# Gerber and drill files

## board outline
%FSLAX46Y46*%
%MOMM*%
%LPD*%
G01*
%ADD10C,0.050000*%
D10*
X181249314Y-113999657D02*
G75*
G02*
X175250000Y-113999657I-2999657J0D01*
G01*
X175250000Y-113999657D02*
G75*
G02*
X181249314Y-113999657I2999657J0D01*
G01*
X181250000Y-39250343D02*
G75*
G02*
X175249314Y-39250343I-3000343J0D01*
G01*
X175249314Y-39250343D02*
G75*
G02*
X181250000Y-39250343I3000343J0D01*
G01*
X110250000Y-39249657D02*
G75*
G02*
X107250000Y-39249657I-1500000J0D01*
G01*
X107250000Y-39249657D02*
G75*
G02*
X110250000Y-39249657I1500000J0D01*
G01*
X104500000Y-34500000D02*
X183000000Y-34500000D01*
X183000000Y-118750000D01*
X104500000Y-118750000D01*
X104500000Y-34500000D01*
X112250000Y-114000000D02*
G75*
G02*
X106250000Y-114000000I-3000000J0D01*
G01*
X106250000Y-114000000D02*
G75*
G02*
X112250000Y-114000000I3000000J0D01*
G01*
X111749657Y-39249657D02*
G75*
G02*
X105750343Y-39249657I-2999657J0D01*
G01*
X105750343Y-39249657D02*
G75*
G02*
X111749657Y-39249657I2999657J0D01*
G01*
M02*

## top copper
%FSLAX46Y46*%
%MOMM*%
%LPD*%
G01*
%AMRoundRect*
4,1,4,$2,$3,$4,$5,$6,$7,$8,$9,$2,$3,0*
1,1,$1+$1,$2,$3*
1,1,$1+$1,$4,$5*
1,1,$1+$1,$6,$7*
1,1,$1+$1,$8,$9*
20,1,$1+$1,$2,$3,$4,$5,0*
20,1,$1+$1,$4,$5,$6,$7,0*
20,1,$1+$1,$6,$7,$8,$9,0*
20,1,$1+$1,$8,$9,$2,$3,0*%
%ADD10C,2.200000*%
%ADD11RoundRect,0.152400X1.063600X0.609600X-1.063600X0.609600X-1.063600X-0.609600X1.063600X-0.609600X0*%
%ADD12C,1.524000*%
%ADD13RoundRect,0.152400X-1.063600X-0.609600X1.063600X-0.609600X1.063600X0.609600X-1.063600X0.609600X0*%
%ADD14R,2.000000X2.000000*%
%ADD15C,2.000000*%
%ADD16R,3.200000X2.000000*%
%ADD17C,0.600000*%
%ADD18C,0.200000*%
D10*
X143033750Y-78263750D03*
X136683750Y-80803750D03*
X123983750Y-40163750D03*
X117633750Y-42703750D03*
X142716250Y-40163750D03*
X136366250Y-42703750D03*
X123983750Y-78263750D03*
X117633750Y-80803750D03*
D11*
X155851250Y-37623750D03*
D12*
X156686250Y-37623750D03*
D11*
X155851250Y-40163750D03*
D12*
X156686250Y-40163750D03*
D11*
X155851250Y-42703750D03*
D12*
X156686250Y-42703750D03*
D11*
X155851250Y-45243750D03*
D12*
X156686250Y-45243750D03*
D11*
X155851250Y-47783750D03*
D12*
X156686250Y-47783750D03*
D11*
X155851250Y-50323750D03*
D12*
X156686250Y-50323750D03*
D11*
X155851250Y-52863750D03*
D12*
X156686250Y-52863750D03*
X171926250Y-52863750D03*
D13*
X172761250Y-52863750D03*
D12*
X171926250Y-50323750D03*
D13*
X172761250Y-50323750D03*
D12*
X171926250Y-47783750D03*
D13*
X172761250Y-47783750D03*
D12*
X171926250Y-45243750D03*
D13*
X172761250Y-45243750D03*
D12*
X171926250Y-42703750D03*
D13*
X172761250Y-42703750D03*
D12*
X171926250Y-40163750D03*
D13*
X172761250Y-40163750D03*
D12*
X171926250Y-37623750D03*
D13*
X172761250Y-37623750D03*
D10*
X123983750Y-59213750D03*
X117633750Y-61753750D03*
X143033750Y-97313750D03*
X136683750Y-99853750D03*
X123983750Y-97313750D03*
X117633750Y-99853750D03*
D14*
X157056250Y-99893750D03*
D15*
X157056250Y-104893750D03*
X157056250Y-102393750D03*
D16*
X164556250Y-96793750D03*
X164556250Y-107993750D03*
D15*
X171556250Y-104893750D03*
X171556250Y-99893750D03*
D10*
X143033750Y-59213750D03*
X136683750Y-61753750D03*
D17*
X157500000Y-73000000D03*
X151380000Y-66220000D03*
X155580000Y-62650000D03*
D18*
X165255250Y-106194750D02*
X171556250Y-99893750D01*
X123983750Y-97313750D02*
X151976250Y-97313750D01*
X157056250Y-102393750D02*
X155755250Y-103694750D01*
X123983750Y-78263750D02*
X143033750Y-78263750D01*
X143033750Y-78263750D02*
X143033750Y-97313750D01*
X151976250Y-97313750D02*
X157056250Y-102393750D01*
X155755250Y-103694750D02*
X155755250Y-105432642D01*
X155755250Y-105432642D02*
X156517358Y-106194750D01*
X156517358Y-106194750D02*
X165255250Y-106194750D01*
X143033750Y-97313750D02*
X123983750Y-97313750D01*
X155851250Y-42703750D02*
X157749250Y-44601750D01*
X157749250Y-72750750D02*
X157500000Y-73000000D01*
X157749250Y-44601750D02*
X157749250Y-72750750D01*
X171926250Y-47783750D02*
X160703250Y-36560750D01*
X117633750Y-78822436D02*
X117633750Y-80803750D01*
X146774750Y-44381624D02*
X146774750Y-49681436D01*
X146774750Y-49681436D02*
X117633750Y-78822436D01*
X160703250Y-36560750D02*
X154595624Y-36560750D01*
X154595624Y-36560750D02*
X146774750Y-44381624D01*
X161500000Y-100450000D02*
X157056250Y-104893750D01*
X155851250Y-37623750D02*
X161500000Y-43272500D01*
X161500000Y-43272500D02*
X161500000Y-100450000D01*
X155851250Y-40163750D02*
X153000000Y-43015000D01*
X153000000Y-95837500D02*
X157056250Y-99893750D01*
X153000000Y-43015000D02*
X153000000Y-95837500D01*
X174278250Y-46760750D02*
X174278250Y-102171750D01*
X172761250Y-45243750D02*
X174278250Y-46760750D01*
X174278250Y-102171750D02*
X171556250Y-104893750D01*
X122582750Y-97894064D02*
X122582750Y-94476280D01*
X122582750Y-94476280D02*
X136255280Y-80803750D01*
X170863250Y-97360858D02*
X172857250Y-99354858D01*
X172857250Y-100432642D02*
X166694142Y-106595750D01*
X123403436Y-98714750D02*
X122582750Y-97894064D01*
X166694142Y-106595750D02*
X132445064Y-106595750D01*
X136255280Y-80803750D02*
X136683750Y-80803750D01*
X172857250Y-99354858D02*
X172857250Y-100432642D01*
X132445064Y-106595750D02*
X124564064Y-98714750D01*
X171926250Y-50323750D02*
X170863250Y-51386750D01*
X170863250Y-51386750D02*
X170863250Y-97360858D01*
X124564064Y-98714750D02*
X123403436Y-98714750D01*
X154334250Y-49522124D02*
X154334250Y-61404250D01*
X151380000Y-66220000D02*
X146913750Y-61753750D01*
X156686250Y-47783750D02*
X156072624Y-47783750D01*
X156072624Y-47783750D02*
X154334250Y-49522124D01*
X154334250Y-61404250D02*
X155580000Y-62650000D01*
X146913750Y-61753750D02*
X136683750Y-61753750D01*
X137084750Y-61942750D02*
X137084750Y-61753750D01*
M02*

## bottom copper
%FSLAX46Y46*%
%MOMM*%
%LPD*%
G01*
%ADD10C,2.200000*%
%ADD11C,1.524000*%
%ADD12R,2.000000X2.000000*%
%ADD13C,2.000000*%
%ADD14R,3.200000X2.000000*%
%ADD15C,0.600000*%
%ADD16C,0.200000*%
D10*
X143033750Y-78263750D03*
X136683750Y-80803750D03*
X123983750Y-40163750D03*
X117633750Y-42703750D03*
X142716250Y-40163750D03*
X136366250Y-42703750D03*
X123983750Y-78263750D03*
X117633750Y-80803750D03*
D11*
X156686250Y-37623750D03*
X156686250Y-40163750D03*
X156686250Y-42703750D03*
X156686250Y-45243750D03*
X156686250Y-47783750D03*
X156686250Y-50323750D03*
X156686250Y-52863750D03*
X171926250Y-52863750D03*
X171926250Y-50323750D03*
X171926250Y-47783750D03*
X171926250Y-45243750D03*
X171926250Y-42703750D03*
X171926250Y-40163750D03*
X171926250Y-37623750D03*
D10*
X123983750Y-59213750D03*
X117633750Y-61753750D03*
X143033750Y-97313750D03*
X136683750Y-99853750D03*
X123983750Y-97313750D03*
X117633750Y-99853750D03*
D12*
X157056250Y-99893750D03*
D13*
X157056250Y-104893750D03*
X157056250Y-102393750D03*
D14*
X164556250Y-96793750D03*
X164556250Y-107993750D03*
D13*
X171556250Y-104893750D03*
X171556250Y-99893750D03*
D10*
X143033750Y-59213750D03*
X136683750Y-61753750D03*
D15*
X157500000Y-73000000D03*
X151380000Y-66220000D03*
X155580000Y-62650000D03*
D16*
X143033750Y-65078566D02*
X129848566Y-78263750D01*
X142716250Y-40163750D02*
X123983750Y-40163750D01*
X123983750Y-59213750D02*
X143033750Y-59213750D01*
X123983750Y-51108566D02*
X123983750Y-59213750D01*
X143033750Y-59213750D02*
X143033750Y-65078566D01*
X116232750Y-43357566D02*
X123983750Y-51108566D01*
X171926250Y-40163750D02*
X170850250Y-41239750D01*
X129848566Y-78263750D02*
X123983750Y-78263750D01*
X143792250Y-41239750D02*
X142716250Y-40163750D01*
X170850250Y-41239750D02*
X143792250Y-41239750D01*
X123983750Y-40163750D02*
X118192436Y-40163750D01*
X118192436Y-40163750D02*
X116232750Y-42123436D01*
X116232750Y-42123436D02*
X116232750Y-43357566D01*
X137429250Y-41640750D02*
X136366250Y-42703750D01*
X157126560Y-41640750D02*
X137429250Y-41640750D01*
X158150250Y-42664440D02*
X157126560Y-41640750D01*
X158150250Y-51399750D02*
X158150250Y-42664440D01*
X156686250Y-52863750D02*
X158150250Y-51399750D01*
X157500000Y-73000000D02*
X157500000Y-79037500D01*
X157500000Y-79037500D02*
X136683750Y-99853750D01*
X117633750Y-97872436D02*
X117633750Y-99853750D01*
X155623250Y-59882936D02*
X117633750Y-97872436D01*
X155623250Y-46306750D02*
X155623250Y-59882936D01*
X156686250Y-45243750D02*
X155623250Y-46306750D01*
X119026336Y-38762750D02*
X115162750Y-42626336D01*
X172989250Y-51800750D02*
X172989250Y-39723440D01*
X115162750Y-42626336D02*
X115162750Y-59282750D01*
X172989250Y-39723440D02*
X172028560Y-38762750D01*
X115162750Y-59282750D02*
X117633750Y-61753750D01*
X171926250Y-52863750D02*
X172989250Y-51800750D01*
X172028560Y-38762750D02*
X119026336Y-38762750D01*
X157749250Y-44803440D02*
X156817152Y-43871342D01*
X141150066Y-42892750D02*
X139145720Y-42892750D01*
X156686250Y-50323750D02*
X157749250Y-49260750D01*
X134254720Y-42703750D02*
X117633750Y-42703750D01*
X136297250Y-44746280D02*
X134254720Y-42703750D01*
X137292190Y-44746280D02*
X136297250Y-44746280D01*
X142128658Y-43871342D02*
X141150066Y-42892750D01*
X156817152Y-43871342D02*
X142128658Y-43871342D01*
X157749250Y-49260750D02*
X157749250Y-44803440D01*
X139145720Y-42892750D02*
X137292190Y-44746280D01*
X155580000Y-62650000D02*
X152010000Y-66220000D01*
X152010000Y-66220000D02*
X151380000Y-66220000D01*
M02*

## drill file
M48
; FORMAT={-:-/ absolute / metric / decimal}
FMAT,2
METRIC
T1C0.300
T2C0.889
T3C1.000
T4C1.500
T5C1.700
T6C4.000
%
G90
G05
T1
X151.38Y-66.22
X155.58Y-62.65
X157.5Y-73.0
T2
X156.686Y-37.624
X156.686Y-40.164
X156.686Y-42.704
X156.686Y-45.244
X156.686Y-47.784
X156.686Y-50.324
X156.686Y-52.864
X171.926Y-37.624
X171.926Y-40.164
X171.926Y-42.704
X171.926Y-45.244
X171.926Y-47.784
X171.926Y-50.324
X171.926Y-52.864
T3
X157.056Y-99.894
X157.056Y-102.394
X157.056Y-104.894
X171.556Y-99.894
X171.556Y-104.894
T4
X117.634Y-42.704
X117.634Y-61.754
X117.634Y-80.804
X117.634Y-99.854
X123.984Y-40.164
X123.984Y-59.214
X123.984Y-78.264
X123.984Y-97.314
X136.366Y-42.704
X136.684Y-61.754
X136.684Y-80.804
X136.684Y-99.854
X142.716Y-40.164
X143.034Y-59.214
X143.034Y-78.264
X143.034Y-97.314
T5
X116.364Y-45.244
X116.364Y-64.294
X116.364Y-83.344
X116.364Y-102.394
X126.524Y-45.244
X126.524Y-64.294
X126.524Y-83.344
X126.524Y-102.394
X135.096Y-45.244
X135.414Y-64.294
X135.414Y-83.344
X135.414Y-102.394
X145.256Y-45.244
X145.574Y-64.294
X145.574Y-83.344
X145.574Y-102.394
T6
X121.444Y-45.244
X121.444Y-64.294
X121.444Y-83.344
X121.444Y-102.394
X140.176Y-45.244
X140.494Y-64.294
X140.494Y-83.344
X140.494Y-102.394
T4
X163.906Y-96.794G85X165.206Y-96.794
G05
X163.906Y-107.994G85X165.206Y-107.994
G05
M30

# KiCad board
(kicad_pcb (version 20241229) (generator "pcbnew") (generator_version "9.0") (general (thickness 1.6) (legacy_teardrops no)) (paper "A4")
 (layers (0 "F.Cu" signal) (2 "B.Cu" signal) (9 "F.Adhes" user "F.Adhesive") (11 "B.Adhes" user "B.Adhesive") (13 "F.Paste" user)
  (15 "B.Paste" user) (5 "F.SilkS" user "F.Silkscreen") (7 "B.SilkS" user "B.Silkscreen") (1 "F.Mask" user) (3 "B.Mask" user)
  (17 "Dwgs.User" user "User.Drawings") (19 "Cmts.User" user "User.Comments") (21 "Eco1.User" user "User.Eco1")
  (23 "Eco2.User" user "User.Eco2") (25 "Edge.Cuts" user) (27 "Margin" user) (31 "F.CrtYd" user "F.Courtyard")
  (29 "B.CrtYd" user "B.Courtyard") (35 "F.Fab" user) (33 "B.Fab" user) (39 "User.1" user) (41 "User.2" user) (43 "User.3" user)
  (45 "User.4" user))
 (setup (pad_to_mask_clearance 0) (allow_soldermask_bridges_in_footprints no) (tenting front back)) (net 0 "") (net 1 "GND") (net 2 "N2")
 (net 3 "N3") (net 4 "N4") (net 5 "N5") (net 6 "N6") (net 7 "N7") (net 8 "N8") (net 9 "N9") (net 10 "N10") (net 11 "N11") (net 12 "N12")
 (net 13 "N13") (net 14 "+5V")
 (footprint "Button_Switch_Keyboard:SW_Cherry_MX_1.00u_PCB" (layer "F.Cu") (at 143.03375 78.26375)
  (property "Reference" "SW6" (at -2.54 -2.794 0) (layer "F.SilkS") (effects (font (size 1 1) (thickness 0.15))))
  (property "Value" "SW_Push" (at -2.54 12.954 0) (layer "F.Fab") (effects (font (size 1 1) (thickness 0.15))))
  (pad "" np_thru_hole circle (at -7.62 5.08) (size 1.7 1.7) (drill 1.7) (layers "*.Cu" "*.Mask"))
  (pad "" np_thru_hole circle (at -2.54 5.08) (size 4 4) (drill 4) (layers "*.Cu" "*.Mask"))
  (pad "" np_thru_hole circle (at 2.54 5.08) (size 1.7 1.7) (drill 1.7) (layers "*.Cu" "*.Mask"))
  (pad "1" thru_hole circle (at 0 0) (size 2.2 2.2) (drill 1.5) (layers "*.Cu" "*.Mask") (remove_unused_layers no) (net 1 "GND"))
  (pad "2" thru_hole circle (at -6.35 2.54) (size 2.2 2.2) (drill 1.5) (layers "*.Cu" "*.Mask") (remove_unused_layers no) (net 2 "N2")))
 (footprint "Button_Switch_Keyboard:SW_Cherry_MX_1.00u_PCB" (layer "F.Cu") (at 123.98375 40.16375)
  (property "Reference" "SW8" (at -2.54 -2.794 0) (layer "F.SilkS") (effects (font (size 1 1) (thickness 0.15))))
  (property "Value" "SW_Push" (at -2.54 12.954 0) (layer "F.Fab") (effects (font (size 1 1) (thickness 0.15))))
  (pad "" np_thru_hole circle (at -7.62 5.08) (size 1.7 1.7) (drill 1.7) (layers "*.Cu" "*.Mask"))
  (pad "" np_thru_hole circle (at -2.54 5.08) (size 4 4) (drill 4) (layers "*.Cu" "*.Mask"))
  (pad "" np_thru_hole circle (at 2.54 5.08) (size 1.7 1.7) (drill 1.7) (layers "*.Cu" "*.Mask"))
  (pad "1" thru_hole circle (at 0 0) (size 2.2 2.2) (drill 1.5) (layers "*.Cu" "*.Mask") (remove_unused_layers no) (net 1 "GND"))
  (pad "2" thru_hole circle (at -6.35 2.54) (size 2.2 2.2) (drill 1.5) (layers "*.Cu" "*.Mask") (remove_unused_layers no) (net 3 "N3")))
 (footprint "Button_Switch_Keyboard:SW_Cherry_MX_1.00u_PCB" (layer "F.Cu") (at 142.71625 40.16375)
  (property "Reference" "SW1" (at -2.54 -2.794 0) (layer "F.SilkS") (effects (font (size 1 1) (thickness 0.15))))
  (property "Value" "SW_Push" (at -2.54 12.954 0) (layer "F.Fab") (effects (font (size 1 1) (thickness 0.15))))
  (pad "" np_thru_hole circle (at -7.62 5.08) (size 1.7 1.7) (drill 1.7) (layers "*.Cu" "*.Mask"))
  (pad "" np_thru_hole circle (at -2.54 5.08) (size 4 4) (drill 4) (layers "*.Cu" "*.Mask"))
  (pad "" np_thru_hole circle (at 2.54 5.08) (size 1.7 1.7) (drill 1.7) (layers "*.Cu" "*.Mask"))
  (pad "1" thru_hole circle (at 0 0) (size 2.2 2.2) (drill 1.5) (layers "*.Cu" "*.Mask") (remove_unused_layers no) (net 1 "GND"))
  (pad "2" thru_hole circle (at -6.35 2.54) (size 2.2 2.2) (drill 1.5) (layers "*.Cu" "*.Mask") (remove_unused_layers no) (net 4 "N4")))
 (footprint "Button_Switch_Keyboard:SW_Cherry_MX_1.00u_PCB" (layer "F.Cu") (at 123.98375 78.26375)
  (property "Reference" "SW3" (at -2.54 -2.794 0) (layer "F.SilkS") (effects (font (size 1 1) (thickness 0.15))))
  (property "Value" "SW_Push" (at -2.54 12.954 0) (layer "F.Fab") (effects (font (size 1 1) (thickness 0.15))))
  (pad "" np_thru_hole circle (at -7.62 5.08) (size 1.7 1.7) (drill 1.7) (layers "*.Cu" "*.Mask"))
  (pad "" np_thru_hole circle (at -2.54 5.08) (size 4 4) (drill 4) (layers "*.Cu" "*.Mask"))
  (pad "" np_thru_hole circle (at 2.54 5.08) (size 1.7 1.7) (drill 1.7) (layers "*.Cu" "*.Mask"))
  (pad "1" thru_hole circle (at 0 0) (size 2.2 2.2) (drill 1.5) (layers "*.Cu" "*.Mask") (remove_unused_layers no) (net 1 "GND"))
  (pad "2" thru_hole circle (at -6.35 2.54) (size 2.2 2.2) (drill 1.5) (layers "*.Cu" "*.Mask") (remove_unused_layers no) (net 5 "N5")))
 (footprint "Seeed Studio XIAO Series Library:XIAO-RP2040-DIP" (layer "F.Cu") (at 164.30625 45.24375)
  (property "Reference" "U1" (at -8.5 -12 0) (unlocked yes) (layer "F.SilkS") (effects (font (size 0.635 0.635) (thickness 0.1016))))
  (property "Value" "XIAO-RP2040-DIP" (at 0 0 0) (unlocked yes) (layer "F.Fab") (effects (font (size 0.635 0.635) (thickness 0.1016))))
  (pad "1" smd roundrect (at -8.455 -7.62 180) (size 2.432 1.524) (layers "F.Cu" "F.Mask") (roundrect_rratio 0.1) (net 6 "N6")
   (thermal_bridge_angle 45))
  (pad "1" thru_hole circle (at -7.62 -7.62 180) (size 1.524 1.524) (drill 0.889) (layers "*.Cu" "*.Mask") (remove_unused_layers no)
   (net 6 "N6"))
  (pad "2" smd roundrect (at -8.455 -5.08 180) (size 2.432 1.524) (layers "F.Cu" "F.Mask") (roundrect_rratio 0.1) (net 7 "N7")
   (thermal_bridge_angle 45))
  (pad "2" thru_hole circle (at -7.62 -5.08 180) (size 1.524 1.524) (drill 0.889) (layers "*.Cu" "*.Mask") (remove_unused_layers no)
   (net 7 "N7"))
  (pad "3" smd roundrect (at -8.455 -2.54 180) (size 2.432 1.524) (layers "F.Cu" "F.Mask") (roundrect_rratio 0.1) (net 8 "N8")
   (thermal_bridge_angle 45))
  (pad "3" thru_hole circle (at -7.62 -2.54 180) (size 1.524 1.524) (drill 0.889) (layers "*.Cu" "*.Mask") (remove_unused_layers no)
   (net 8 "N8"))
  (pad "4" smd roundrect (at -8.455 0 180) (size 2.432 1.524) (layers "F.Cu" "F.Mask") (roundrect_rratio 0.1) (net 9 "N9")
   (thermal_bridge_angle 45))
  (pad "4" thru_hole circle (at -7.62 0 180) (size 1.524 1.524) (drill 0.889) (layers "*.Cu" "*.Mask") (remove_unused_layers no)
   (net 9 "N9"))
  (pad "5" smd roundrect (at -8.455 2.54 180) (size 2.432 1.524) (layers "F.Cu" "F.Mask") (roundrect_rratio 0.1) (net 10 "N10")
   (thermal_bridge_angle 45))
  (pad "5" thru_hole circle (at -7.62 2.54 180) (size 1.524 1.524) (drill 0.889) (layers "*.Cu" "*.Mask") (remove_unused_layers no)
   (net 10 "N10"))
  (pad "6" smd roundrect (at -8.455 5.08 180) (size 2.432 1.524) (layers "F.Cu" "F.Mask") (roundrect_rratio 0.1) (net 3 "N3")
   (thermal_bridge_angle 45))
  (pad "6" thru_hole circle (at -7.62 5.08 180) (size 1.524 1.524) (drill 0.889) (layers "*.Cu" "*.Mask") (remove_unused_layers no)
   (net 3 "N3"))
  (pad "7" smd roundrect (at -8.455 7.62 180) (size 2.432 1.524) (layers "F.Cu" "F.Mask") (roundrect_rratio 0.1) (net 4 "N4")
   (thermal_bridge_angle 45))
  (pad "7" thru_hole circle (at -7.62 7.62 180) (size 1.524 1.524) (drill 0.889) (layers "*.Cu" "*.Mask") (remove_unused_layers no)
   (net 4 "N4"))
  (pad "8" thru_hole circle (at 7.62 7.62) (size 1.524 1.524) (drill 0.889) (layers "*.Cu" "*.Mask") (remove_unused_layers no)
   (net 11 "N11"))
  (pad "8" smd roundrect (at 8.455 7.62) (size 2.432 1.524) (layers "F.Cu" "F.Mask") (roundrect_rratio 0.1) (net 11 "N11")
   (thermal_bridge_angle 45))
  (pad "9" thru_hole circle (at 7.62 5.08) (size 1.524 1.524) (drill 0.889) (layers "*.Cu" "*.Mask") (remove_unused_layers no) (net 2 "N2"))
  (pad "9" smd roundrect (at 8.455 5.08) (size 2.432 1.524) (layers "F.Cu" "F.Mask") (roundrect_rratio 0.1) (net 2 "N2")
   (thermal_bridge_angle 45))
  (pad "10" thru_hole circle (at 7.62 2.54) (size 1.524 1.524) (drill 0.889) (layers "*.Cu" "*.Mask") (remove_unused_layers no) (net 5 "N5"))
  (pad "10" smd roundrect (at 8.455 2.54) (size 2.432 1.524) (layers "F.Cu" "F.Mask") (roundrect_rratio 0.1) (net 5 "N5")
   (thermal_bridge_angle 45))
  (pad "11" thru_hole circle (at 7.62 0) (size 1.524 1.524) (drill 0.889) (layers "*.Cu" "*.Mask") (remove_unused_layers no) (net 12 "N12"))
  (pad "11" smd roundrect (at 8.455 0) (size 2.432 1.524) (layers "F.Cu" "F.Mask") (roundrect_rratio 0.1) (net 12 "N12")
   (thermal_bridge_angle 45))
  (pad "12" thru_hole circle (at 7.62 -2.54) (size 1.524 1.524) (drill 0.889) (layers "*.Cu" "*.Mask") (remove_unused_layers no)
   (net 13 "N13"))
  (pad "12" smd roundrect (at 8.455 -2.54) (size 2.432 1.524) (layers "F.Cu" "F.Mask") (roundrect_rratio 0.1) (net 13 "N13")
   (thermal_bridge_angle 45))
  (pad "13" thru_hole circle (at 7.62 -5.08) (size 1.524 1.524) (drill 0.889) (layers "*.Cu" "*.Mask") (remove_unused_layers no)
   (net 1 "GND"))
  (pad "13" smd roundrect (at 8.455 -5.08) (size 2.432 1.524) (layers "F.Cu" "F.Mask") (roundrect_rratio 0.1) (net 1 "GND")
   (thermal_bridge_angle 45))
  (pad "14" thru_hole circle (at 7.62 -7.62) (size 1.524 1.524) (drill 0.889) (layers "*.Cu" "*.Mask") (remove_unused_layers no)
   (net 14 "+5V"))
  (pad "14" smd roundrect (at 8.455 -7.62) (size 2.432 1.524) (layers "F.Cu" "F.Mask") (roundrect_rratio 0.1) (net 14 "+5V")
   (thermal_bridge_angle 45)))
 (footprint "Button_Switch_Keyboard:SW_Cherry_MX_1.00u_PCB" (layer "F.Cu") (at 123.98375 59.21375)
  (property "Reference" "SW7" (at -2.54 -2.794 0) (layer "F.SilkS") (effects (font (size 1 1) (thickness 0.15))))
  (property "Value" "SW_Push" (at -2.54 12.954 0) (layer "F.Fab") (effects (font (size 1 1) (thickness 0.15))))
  (pad "" np_thru_hole circle (at -7.62 5.08) (size 1.7 1.7) (drill 1.7) (layers "*.Cu" "*.Mask"))
  (pad "" np_thru_hole circle (at -2.54 5.08) (size 4 4) (drill 4) (layers "*.Cu" "*.Mask"))
  (pad "" np_thru_hole circle (at 2.54 5.08) (size 1.7 1.7) (drill 1.7) (layers "*.Cu" "*.Mask"))
  (pad "1" thru_hole circle (at 0 0) (size 2.2 2.2) (drill 1.5) (layers "*.Cu" "*.Mask") (remove_unused_layers no) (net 1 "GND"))
  (pad "2" thru_hole circle (at -6.35 2.54) (size 2.2 2.2) (drill 1.5) (layers "*.Cu" "*.Mask") (remove_unused_layers no) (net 11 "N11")))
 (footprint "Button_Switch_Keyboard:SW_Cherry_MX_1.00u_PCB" (layer "F.Cu") (at 143.03375 97.31375)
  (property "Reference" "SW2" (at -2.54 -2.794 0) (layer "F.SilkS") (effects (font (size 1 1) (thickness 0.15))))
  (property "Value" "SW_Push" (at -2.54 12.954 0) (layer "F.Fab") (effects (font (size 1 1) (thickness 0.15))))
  (pad "" np_thru_hole circle (at -7.62 5.08) (size 1.7 1.7) (drill 1.7) (layers "*.Cu" "*.Mask"))
  (pad "" np_thru_hole circle (at -2.54 5.08) (size 4 4) (drill 4) (layers "*.Cu" "*.Mask"))
  (pad "" np_thru_hole circle (at 2.54 5.08) (size 1.7 1.7) (drill 1.7) (layers "*.Cu" "*.Mask"))
  (pad "1" thru_hole circle (at 0 0) (size 2.2 2.2) (drill 1.5) (layers "*.Cu" "*.Mask") (remove_unused_layers no) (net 1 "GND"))
  (pad "2" thru_hole circle (at -6.35 2.54) (size 2.2 2.2) (drill 1.5) (layers "*.Cu" "*.Mask") (remove_unused_layers no) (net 8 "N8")))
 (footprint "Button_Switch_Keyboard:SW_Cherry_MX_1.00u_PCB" (layer "F.Cu") (at 123.98375 97.31375)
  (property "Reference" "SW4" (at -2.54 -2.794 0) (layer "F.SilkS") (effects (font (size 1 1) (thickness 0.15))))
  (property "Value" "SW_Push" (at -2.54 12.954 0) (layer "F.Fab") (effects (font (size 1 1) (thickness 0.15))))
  (pad "" np_thru_hole circle (at -7.62 5.08) (size 1.7 1.7) (drill 1.7) (layers "*.Cu" "*.Mask"))
  (pad "" np_thru_hole circle (at -2.54 5.08) (size 4 4) (drill 4) (layers "*.Cu" "*.Mask"))
  (pad "" np_thru_hole circle (at 2.54 5.08) (size 1.7 1.7) (drill 1.7) (layers "*.Cu" "*.Mask"))
  (pad "1" thru_hole circle (at 0 0) (size 2.2 2.2) (drill 1.5) (layers "*.Cu" "*.Mask") (remove_unused_layers no) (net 1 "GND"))
  (pad "2" thru_hole circle (at -6.35 2.54) (size 2.2 2.2) (drill 1.5) (layers "*.Cu" "*.Mask") (remove_unused_layers no) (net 9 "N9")))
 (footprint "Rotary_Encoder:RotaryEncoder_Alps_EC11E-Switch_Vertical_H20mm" (layer "F.Cu") (at 157.05625 99.89375)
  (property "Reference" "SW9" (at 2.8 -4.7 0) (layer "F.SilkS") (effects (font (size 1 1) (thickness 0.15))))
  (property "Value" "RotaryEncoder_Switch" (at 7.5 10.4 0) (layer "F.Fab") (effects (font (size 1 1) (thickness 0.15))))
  (pad "A" thru_hole rect (at 0 0) (size 2 2) (drill 1) (layers "*.Cu" "*.Mask") (remove_unused_layers no) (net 7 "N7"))
  (pad "B" thru_hole circle (at 0 5) (size 2 2) (drill 1) (layers "*.Cu" "*.Mask") (remove_unused_layers no) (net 6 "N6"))
  (pad "C" thru_hole circle (at 0 2.5) (size 2 2) (drill 1) (layers "*.Cu" "*.Mask") (remove_unused_layers no) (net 1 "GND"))
  (pad "MP" thru_hole rect (at 7.5 -3.1) (size 3.2 2) (drill oval 2.8 1.5) (layers "*.Cu" "*.Mask") (remove_unused_layers no))
  (pad "MP" thru_hole rect (at 7.5 8.1) (size 3.2 2) (drill oval 2.8 1.5) (layers "*.Cu" "*.Mask") (remove_unused_layers no))
  (pad "S1" thru_hole circle (at 14.5 5) (size 2 2) (drill 1) (layers "*.Cu" "*.Mask") (remove_unused_layers no) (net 12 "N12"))
  (pad "S2" thru_hole circle (at 14.5 0) (size 2 2) (drill 1) (layers "*.Cu" "*.Mask") (remove_unused_layers no) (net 1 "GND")))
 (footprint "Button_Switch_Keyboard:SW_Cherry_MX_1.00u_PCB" (layer "F.Cu") (at 143.03375 59.21375)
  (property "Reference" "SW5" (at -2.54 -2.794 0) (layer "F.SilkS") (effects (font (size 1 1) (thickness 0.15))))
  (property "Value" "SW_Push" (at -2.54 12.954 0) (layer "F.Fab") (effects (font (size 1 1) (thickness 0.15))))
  (pad "" np_thru_hole circle (at -7.62 5.08) (size 1.7 1.7) (drill 1.7) (layers "*.Cu" "*.Mask"))
  (pad "" np_thru_hole circle (at -2.54 5.08) (size 4 4) (drill 4) (layers "*.Cu" "*.Mask"))
  (pad "" np_thru_hole circle (at 2.54 5.08) (size 1.7 1.7) (drill 1.7) (layers "*.Cu" "*.Mask"))
  (pad "1" thru_hole circle (at 0 0) (size 2.2 2.2) (drill 1.5) (layers "*.Cu" "*.Mask") (remove_unused_layers no) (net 1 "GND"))
  (pad "2" thru_hole circle (at -6.35 2.54) (size 2.2 2.2) (drill 1.5) (layers "*.Cu" "*.Mask") (remove_unused_layers no) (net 10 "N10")))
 (gr_circle (center 178.249657 113.999657) (end 175.25 113.999657) (stroke (width 0.05) (type default)) (fill no) (layer "Edge.Cuts"))
 (gr_circle (center 178.249657 39.250343) (end 181.25 39.250343) (stroke (width 0.05) (type default)) (fill no) (layer "Edge.Cuts"))
 (gr_circle (center 108.75 39.249657) (end 107.25 39.249657) (stroke (width 0.05) (type default)) (fill no) (layer "Edge.Cuts"))
 (gr_rect (start 104.5 34.5) (end 183 118.75) (stroke (width 0.05) (type default)) (fill no) (layer "Edge.Cuts"))
 (gr_circle (center 109.25 114) (end 112.25 114) (stroke (width 0.05) (type default)) (fill no) (layer "Edge.Cuts"))
 (gr_circle (center 108.75 39.249657) (end 111.749657 39.249657) (stroke (width 0.05) (type default)) (fill no) (layer "Edge.Cuts"))
 (segment (start 165.25525 106.19475) (end 171.55625 99.89375) (width 0.2) (layer "F.Cu") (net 1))
 (segment (start 123.98375 97.31375) (end 151.97625 97.31375) (width 0.2) (layer "F.Cu") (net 1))
 (segment (start 157.05625 102.39375) (end 155.75525 103.69475) (width 0.2) (layer "F.Cu") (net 1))
 (segment (start 123.98375 78.26375) (end 143.03375 78.26375) (width 0.2) (layer "F.Cu") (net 1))
 (segment (start 143.03375 78.26375) (end 143.03375 97.31375) (width 0.2) (layer "F.Cu") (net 1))
 (segment (start 151.97625 97.31375) (end 157.05625 102.39375) (width 0.2) (layer "F.Cu") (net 1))
 (segment (start 155.75525 103.69475) (end 155.75525 105.432642) (width 0.2) (layer "F.Cu") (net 1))
 (segment (start 155.75525 105.432642) (end 156.517358 106.19475) (width 0.2) (layer "F.Cu") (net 1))
 (segment (start 156.517358 106.19475) (end 165.25525 106.19475) (width 0.2) (layer "F.Cu") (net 1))
 (segment (start 143.03375 97.31375) (end 123.98375 97.31375) (width 0.2) (layer "F.Cu") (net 1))
 (segment (start 143.03375 65.078566) (end 129.848566 78.26375) (width 0.2) (layer "B.Cu") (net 1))
 (segment (start 142.71625 40.16375) (end 123.98375 40.16375) (width 0.2) (layer "B.Cu") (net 1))
 (segment (start 123.98375 59.21375) (end 143.03375 59.21375) (width 0.2) (layer "B.Cu") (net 1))
 (segment (start 123.98375 51.108566) (end 123.98375 59.21375) (width 0.2) (layer "B.Cu") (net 1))
 (segment (start 143.03375 59.21375) (end 143.03375 65.078566) (width 0.2) (layer "B.Cu") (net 1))
 (segment (start 116.23275 43.357566) (end 123.98375 51.108566) (width 0.2) (layer "B.Cu") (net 1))
 (segment (start 171.92625 40.16375) (end 170.85025 41.23975) (width 0.2) (layer "B.Cu") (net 1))
 (segment (start 129.848566 78.26375) (end 123.98375 78.26375) (width 0.2) (layer "B.Cu") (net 1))
 (segment (start 143.79225 41.23975) (end 142.71625 40.16375) (width 0.2) (layer "B.Cu") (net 1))
 (segment (start 170.85025 41.23975) (end 143.79225 41.23975) (width 0.2) (layer "B.Cu") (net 1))
 (segment (start 123.98375 40.16375) (end 118.192436 40.16375) (width 0.2) (layer "B.Cu") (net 1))
 (segment (start 118.192436 40.16375) (end 116.23275 42.123436) (width 0.2) (layer "B.Cu") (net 1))
 (segment (start 116.23275 42.123436) (end 116.23275 43.357566) (width 0.2) (layer "B.Cu") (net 1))
 (segment (start 137.42925 41.64075) (end 136.36625 42.70375) (width 0.2) (layer "B.Cu") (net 4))
 (segment (start 157.12656 41.64075) (end 137.42925 41.64075) (width 0.2) (layer "B.Cu") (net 4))
 (segment (start 158.15025 42.66444) (end 157.12656 41.64075) (width 0.2) (layer "B.Cu") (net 4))
 (segment (start 158.15025 51.39975) (end 158.15025 42.66444) (width 0.2) (layer "B.Cu") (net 4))
 (segment (start 156.68625 52.86375) (end 158.15025 51.39975) (width 0.2) (layer "B.Cu") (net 4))
 (segment (start 155.85125 42.70375) (end 157.74925 44.60175) (width 0.2) (layer "F.Cu") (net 8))
 (segment (start 157.74925 72.75075) (end 157.5 73) (width 0.2) (layer "F.Cu") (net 8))
 (segment (start 157.74925 44.60175) (end 157.74925 72.75075) (width 0.2) (layer "F.Cu") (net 8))
 (via (at 157.5 73) (size 0.6) (drill 0.3) (layers "F.Cu" "B.Cu") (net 8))
 (segment (start 157.5 73) (end 157.5 79.0375) (width 0.2) (layer "B.Cu") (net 8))
 (segment (start 157.5 79.0375) (end 136.68375 99.85375) (width 0.2) (layer "B.Cu") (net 8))
 (segment (start 171.92625 47.78375) (end 160.70325 36.56075) (width 0.2) (layer "F.Cu") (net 5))
 (segment (start 117.63375 78.822436) (end 117.63375 80.80375) (width 0.2) (layer "F.Cu") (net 5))
 (segment (start 146.77475 44.381624) (end 146.77475 49.681436) (width 0.2) (layer "F.Cu") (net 5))
 (segment (start 146.77475 49.681436) (end 117.63375 78.822436) (width 0.2) (layer "F.Cu") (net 5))
 (segment (start 160.70325 36.56075) (end 154.595624 36.56075) (width 0.2) (layer "F.Cu") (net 5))
 (segment (start 154.595624 36.56075) (end 146.77475 44.381624) (width 0.2) (layer "F.Cu") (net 5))
 (segment (start 117.63375 97.872436) (end 117.63375 99.85375) (width 0.2) (layer "B.Cu") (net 9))
 (segment (start 155.62325 59.882936) (end 117.63375 97.872436) (width 0.2) (layer "B.Cu") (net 9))
 (segment (start 155.62325 46.30675) (end 155.62325 59.882936) (width 0.2) (layer "B.Cu") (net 9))
 (segment (start 156.68625 45.24375) (end 155.62325 46.30675) (width 0.2) (layer "B.Cu") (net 9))
 (segment (start 119.026336 38.76275) (end 115.16275 42.626336) (width 0.2) (layer "B.Cu") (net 11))
 (segment (start 172.98925 51.80075) (end 172.98925 39.72344) (width 0.2) (layer "B.Cu") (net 11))
 (segment (start 115.16275 42.626336) (end 115.16275 59.28275) (width 0.2) (layer "B.Cu") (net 11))
 (segment (start 172.98925 39.72344) (end 172.02856 38.76275) (width 0.2) (layer "B.Cu") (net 11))
 (segment (start 115.16275 59.28275) (end 117.63375 61.75375) (width 0.2) (layer "B.Cu") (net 11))
 (segment (start 171.92625 52.86375) (end 172.98925 51.80075) (width 0.2) (layer "B.Cu") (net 11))
 (segment (start 172.02856 38.76275) (end 119.026336 38.76275) (width 0.2) (layer "B.Cu") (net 11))
 (segment (start 157.74925 44.80344) (end 156.817152 43.871342) (width 0.2) (layer "B.Cu") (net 3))
 (segment (start 141.150066 42.89275) (end 139.14572 42.89275) (width 0.2) (layer "B.Cu") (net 3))
 (segment (start 156.68625 50.32375) (end 157.74925 49.26075) (width 0.2) (layer "B.Cu") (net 3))
 (segment (start 134.25472 42.70375) (end 117.63375 42.70375) (width 0.2) (layer "B.Cu") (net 3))
 (segment (start 136.29725 44.74628) (end 134.25472 42.70375) (width 0.2) (layer "B.Cu") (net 3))
 (segment (start 137.29219 44.74628) (end 136.29725 44.74628) (width 0.2) (layer "B.Cu") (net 3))
 (segment (start 142.128658 43.871342) (end 141.150066 42.89275) (width 0.2) (layer "B.Cu") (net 3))
 (segment (start 156.817152 43.871342) (end 142.128658 43.871342) (width 0.2) (layer "B.Cu") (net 3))
 (segment (start 157.74925 49.26075) (end 157.74925 44.80344) (width 0.2) (layer "B.Cu") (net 3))
 (segment (start 139.14572 42.89275) (end 137.29219 44.74628) (width 0.2) (layer "B.Cu") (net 3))
 (segment (start 161.5 100.45) (end 157.05625 104.89375) (width 0.2) (layer "F.Cu") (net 6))
 (segment (start 155.85125 37.62375) (end 161.5 43.2725) (width 0.2) (layer "F.Cu") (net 6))
 (segment (start 161.5 43.2725) (end 161.5 100.45) (width 0.2) (layer "F.Cu") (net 6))
 (segment (start 155.85125 40.16375) (end 153 43.015) (width 0.2) (layer "F.Cu") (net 7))
 (segment (start 153 95.8375) (end 157.05625 99.89375) (width 0.2) (layer "F.Cu") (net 7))
 (segment (start 153 43.015) (end 153 95.8375) (width 0.2) (layer "F.Cu") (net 7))
 (segment (start 174.27825 46.76075) (end 174.27825 102.17175) (width 0.2) (layer "F.Cu") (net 12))
 (segment (start 172.76125 45.24375) (end 174.27825 46.76075) (width 0.2) (layer "F.Cu") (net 12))
 (segment (start 174.27825 102.17175) (end 171.55625 104.89375) (width 0.2) (layer "F.Cu") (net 12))
 (segment (start 122.58275 97.894064) (end 122.58275 94.47628) (width 0.2) (layer "F.Cu") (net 2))
 (segment (start 122.58275 94.47628) (end 136.25528 80.80375) (width 0.2) (layer "F.Cu") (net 2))
 (segment (start 170.86325 97.360858) (end 172.85725 99.354858) (width 0.2) (layer "F.Cu") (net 2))
 (segment (start 172.85725 100.432642) (end 166.694142 106.59575) (width 0.2) (layer "F.Cu") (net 2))
 (segment (start 123.403436 98.71475) (end 122.58275 97.894064) (width 0.2) (layer "F.Cu") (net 2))
 (segment (start 166.694142 106.59575) (end 132.445064 106.59575) (width 0.2) (layer "F.Cu") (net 2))
 (segment (start 136.25528 80.80375) (end 136.68375 80.80375) (width 0.2) (layer "F.Cu") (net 2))
 (segment (start 172.85725 99.354858) (end 172.85725 100.432642) (width 0.2) (layer "F.Cu") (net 2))
 (segment (start 132.445064 106.59575) (end 124.564064 98.71475) (width 0.2) (layer "F.Cu") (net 2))
 (segment (start 171.92625 50.32375) (end 170.86325 51.38675) (width 0.2) (layer "F.Cu") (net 2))
 (segment (start 170.86325 51.38675) (end 170.86325 97.360858) (width 0.2) (layer "F.Cu") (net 2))
 (segment (start 124.564064 98.71475) (end 123.403436 98.71475) (width 0.2) (layer "F.Cu") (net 2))
 (segment (start 154.33425 49.522124) (end 154.33425 61.40425) (width 0.2) (layer "F.Cu") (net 10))
 (segment (start 151.38 66.22) (end 146.91375 61.75375) (width 0.2) (layer "F.Cu") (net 10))
 (segment (start 156.68625 47.78375) (end 156.072624 47.78375) (width 0.2) (layer "F.Cu") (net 10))
 (segment (start 156.072624 47.78375) (end 154.33425 49.522124) (width 0.2) (layer "F.Cu") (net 10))
 (segment (start 154.33425 61.40425) (end 155.58 62.65) (width 0.2) (layer "F.Cu") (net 10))
 (segment (start 146.91375 61.75375) (end 136.68375 61.75375) (width 0.2) (layer "F.Cu") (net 10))
 (segment (start 137.08475 61.94275) (end 137.08475 61.75375) (width 0.2) (layer "F.Cu") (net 10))
 (via (at 151.38 66.22) (size 0.6) (drill 0.3) (layers "F.Cu" "B.Cu") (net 10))
 (via (at 155.58 62.65) (size 0.6) (drill 0.3) (layers "F.Cu" "B.Cu") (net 10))
 (segment (start 155.58 62.65) (end 152.01 66.22) (width 0.2) (layer "B.Cu") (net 10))
 (segment (start 152.01 66.22) (end 151.38 66.22) (width 0.2) (layer "B.Cu") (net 10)))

